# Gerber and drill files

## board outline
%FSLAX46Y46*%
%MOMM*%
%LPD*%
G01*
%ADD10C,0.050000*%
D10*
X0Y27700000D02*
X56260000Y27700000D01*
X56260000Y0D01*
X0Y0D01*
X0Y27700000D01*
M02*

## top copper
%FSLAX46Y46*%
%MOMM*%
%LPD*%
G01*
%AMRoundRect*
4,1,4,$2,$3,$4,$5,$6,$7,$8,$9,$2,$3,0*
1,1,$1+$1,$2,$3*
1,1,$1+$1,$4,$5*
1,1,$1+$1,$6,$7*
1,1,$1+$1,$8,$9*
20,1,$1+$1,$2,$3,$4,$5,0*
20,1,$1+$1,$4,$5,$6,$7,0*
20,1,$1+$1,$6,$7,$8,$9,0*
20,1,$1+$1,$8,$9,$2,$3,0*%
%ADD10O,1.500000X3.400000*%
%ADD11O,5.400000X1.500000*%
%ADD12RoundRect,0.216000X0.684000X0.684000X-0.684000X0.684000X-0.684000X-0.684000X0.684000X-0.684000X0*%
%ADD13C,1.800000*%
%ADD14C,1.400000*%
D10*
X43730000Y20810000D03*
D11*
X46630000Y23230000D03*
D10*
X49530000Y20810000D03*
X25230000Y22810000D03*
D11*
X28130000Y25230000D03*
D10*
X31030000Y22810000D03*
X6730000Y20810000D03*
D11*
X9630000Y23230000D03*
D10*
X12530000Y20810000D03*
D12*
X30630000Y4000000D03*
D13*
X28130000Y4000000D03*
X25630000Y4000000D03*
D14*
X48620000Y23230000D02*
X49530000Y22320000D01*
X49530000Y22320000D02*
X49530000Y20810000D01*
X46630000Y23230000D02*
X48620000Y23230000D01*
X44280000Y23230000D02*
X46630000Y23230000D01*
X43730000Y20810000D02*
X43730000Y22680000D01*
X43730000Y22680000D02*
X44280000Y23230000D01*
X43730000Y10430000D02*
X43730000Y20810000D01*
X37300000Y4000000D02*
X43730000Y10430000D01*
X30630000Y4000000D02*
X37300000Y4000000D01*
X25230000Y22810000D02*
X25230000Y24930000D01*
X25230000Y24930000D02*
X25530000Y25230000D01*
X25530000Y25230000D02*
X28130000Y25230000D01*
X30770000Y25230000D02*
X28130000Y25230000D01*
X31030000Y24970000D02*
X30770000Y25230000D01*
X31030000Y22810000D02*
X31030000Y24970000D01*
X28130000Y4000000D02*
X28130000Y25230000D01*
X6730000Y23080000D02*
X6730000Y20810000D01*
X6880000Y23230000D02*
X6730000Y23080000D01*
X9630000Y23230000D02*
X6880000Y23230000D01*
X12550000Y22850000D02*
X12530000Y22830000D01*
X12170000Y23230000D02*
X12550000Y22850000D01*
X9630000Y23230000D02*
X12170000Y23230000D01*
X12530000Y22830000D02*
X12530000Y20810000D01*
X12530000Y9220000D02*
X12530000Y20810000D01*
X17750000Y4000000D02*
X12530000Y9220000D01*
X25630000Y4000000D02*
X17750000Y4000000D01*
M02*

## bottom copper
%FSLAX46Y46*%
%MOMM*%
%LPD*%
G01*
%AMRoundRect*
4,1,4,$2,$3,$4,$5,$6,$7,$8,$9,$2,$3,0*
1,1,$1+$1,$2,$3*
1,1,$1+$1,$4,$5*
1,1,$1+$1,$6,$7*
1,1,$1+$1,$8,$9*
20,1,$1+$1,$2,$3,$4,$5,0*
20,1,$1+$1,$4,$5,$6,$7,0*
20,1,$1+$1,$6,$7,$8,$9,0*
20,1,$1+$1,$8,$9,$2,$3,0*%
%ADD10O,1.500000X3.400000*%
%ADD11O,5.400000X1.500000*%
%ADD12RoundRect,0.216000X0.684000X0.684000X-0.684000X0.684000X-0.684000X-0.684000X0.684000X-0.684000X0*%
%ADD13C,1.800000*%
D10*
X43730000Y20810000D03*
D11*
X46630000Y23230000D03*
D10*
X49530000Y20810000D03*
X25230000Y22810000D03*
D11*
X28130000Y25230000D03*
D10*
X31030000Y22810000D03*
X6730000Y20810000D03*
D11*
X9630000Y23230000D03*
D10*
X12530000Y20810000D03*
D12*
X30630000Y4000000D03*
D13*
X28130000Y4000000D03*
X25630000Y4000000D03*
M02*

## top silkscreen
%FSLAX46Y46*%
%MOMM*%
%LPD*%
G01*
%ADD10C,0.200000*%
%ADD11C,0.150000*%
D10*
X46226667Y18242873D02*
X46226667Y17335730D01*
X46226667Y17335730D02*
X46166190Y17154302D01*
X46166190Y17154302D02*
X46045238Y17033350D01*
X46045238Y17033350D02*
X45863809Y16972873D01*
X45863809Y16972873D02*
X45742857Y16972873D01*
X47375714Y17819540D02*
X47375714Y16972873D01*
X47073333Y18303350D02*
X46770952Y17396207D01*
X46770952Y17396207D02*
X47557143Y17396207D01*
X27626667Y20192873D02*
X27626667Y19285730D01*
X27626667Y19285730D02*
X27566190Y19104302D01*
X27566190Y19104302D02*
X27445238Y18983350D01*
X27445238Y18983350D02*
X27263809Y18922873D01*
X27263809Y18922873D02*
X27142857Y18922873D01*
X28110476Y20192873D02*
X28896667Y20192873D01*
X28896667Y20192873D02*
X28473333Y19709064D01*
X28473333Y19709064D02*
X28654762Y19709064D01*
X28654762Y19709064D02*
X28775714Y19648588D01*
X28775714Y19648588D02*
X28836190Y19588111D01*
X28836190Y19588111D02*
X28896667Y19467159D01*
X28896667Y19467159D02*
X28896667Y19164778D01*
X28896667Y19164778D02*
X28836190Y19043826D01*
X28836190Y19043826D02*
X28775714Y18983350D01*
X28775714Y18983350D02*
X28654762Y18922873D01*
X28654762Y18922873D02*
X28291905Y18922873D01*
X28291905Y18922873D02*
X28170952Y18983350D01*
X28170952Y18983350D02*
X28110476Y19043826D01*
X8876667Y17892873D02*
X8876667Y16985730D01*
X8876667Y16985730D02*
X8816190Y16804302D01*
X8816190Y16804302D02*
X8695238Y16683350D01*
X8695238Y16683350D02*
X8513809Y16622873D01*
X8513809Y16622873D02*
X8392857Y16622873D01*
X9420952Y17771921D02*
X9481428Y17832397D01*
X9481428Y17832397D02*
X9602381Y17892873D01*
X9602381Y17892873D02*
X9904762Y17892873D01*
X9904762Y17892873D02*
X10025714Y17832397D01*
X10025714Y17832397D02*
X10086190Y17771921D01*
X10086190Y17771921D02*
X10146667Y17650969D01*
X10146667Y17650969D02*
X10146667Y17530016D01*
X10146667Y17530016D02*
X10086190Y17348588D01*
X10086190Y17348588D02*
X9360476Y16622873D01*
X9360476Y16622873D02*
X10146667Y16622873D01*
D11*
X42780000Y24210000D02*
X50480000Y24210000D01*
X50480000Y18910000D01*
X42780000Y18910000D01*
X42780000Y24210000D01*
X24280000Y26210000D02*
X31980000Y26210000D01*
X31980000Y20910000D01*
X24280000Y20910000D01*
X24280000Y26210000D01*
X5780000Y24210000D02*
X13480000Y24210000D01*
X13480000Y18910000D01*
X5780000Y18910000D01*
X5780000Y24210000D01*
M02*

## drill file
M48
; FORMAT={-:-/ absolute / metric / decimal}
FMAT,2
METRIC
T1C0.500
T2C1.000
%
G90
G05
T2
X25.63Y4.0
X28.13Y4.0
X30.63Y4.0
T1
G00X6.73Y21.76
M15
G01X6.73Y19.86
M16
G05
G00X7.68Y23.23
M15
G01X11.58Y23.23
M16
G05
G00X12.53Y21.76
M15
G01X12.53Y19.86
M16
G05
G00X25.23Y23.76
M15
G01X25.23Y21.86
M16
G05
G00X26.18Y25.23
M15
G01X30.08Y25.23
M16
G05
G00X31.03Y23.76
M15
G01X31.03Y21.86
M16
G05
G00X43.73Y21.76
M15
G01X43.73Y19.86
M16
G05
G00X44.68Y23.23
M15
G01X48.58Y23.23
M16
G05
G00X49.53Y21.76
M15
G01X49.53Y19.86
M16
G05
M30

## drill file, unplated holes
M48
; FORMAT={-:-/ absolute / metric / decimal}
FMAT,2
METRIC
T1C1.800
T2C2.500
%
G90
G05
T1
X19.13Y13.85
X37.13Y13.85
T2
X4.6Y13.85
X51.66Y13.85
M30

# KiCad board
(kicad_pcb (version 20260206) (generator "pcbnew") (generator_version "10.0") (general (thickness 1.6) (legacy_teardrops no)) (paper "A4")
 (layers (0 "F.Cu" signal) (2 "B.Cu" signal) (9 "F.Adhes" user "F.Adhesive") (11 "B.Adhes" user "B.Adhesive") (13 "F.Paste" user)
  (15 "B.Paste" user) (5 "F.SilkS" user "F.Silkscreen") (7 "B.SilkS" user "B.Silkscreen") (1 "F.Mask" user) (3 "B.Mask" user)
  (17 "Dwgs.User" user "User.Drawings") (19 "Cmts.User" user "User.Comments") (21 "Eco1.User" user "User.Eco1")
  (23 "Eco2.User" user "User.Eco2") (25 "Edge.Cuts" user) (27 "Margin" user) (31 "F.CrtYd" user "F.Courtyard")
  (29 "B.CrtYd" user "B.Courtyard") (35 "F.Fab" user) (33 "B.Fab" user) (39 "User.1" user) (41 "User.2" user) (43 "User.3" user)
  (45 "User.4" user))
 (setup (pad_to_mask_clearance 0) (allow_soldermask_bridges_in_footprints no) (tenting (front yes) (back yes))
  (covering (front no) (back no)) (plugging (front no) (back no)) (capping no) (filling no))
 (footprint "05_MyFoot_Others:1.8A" (layer "F.Cu") (at 37.13 -13.85)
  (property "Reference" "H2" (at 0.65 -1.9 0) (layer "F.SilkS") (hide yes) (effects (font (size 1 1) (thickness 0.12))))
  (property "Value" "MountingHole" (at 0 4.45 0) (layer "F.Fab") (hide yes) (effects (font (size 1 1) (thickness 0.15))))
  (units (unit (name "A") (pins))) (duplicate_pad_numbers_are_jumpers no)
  (pad "" np_thru_hole circle (at 0 0) (size 1.8 1.8) (drill 1.8) (layers "*.Cu" "*.Mask") (zone_connect 2)))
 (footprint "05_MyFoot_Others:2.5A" (layer "F.Cu") (at 51.66 -13.85)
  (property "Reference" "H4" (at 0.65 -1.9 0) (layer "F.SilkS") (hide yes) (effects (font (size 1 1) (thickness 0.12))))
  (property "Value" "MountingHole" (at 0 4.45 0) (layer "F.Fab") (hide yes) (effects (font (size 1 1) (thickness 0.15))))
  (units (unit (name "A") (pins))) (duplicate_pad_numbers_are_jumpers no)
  (pad "" np_thru_hole circle (at 0 0) (size 2.5 2.5) (drill 2.5) (layers "*.Cu" "*.Mask") (zone_connect 2)))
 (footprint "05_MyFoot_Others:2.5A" (layer "F.Cu") (at 4.6 -13.85)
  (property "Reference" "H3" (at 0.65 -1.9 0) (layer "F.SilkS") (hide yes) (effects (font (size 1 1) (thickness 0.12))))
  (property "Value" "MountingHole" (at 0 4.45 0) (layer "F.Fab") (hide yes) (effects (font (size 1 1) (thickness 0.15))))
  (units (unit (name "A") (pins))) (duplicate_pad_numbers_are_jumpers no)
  (pad "" np_thru_hole circle (at 0 0) (size 2.5 2.5) (drill 2.5) (layers "*.Cu" "*.Mask") (zone_connect 2)))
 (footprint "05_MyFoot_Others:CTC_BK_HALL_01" (layer "F.Cu") (at 28.13 -22.81)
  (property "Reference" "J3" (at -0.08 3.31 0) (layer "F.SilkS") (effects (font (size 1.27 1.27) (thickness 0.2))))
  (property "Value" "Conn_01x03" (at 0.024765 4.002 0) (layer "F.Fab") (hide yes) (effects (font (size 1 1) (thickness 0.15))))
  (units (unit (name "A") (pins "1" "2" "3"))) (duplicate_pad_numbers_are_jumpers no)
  (fp_rect (start -3.85 -3.4) (end 3.85 1.9) (stroke (width 0.15) (type solid)) (fill no) (layer "F.SilkS"))
  (pad "1" thru_hole oval (at -2.9 0) (size 1.5 3.4) (drill oval 0.5 2.4) (layers "*.Cu" "*.Mask") (remove_unused_layers no)
   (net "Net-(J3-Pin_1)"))
  (pad "2" thru_hole oval (at 0 -2.42) (size 5.4 1.5) (drill oval 4.4 0.5) (layers "*.Cu" "*.Mask") (remove_unused_layers no)
   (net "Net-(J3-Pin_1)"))
  (pad "3" thru_hole oval (at 2.9 0) (size 1.5 3.4) (drill oval 0.5 2.4) (layers "*.Cu" "*.Mask") (remove_unused_layers no)
   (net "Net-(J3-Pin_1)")))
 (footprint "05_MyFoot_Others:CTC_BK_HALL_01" (layer "F.Cu") (at 46.63 -20.81)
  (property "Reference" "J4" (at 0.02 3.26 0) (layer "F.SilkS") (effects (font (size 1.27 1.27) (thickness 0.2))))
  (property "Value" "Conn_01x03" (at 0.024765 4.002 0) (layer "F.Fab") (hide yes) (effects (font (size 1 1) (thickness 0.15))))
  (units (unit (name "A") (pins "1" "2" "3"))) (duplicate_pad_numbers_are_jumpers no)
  (fp_rect (start -3.85 -3.4) (end 3.85 1.9) (stroke (width 0.15) (type solid)) (fill no) (layer "F.SilkS"))
  (pad "1" thru_hole oval (at -2.9 0) (size 1.5 3.4) (drill oval 0.5 2.4) (layers "*.Cu" "*.Mask") (remove_unused_layers no)
   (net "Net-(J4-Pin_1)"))
  (pad "2" thru_hole oval (at 0 -2.42) (size 5.4 1.5) (drill oval 4.4 0.5) (layers "*.Cu" "*.Mask") (remove_unused_layers no)
   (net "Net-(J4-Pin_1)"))
  (pad "3" thru_hole oval (at 2.9 0) (size 1.5 3.4) (drill oval 0.5 2.4) (layers "*.Cu" "*.Mask") (remove_unused_layers no)
   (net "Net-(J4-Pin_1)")))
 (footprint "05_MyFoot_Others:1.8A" (layer "F.Cu") (at 19.13 -13.85)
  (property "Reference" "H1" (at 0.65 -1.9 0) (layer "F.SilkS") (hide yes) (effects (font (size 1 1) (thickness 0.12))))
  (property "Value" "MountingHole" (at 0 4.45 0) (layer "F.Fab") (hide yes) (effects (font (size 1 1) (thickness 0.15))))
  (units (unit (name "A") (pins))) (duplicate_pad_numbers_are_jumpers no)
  (pad "" np_thru_hole circle (at 0 0) (size 1.8 1.8) (drill 1.8) (layers "*.Cu" "*.Mask") (zone_connect 2)))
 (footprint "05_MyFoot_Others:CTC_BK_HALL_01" (layer "F.Cu") (at 9.63 -20.81)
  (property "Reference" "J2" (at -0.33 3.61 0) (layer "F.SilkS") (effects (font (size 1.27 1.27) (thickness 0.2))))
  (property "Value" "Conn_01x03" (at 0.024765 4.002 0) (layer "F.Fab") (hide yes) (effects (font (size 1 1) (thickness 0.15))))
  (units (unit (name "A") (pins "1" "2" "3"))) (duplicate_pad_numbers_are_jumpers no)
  (fp_rect (start -3.85 -3.4) (end 3.85 1.9) (stroke (width 0.15) (type solid)) (fill no) (layer "F.SilkS"))
  (pad "1" thru_hole oval (at -2.9 0) (size 1.5 3.4) (drill oval 0.5 2.4) (layers "*.Cu" "*.Mask") (remove_unused_layers no)
   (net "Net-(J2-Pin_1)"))
  (pad "2" thru_hole oval (at 0 -2.42) (size 5.4 1.5) (drill oval 4.4 0.5) (layers "*.Cu" "*.Mask") (remove_unused_layers no)
   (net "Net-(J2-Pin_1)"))
  (pad "3" thru_hole oval (at 2.9 0) (size 1.5 3.4) (drill oval 0.5 2.4) (layers "*.Cu" "*.Mask") (remove_unused_layers no)
   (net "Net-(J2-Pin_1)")))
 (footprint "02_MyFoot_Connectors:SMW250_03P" (layer "B.Cu") (at 28.13 -4 180)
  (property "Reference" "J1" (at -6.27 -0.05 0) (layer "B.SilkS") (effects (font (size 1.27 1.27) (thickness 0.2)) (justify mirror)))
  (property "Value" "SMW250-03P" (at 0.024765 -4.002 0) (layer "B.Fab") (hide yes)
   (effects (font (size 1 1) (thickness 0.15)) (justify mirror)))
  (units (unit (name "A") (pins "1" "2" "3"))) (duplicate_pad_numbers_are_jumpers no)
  (pad "1" thru_hole roundrect (at -2.5 0 180) (size 1.8 1.8) (drill 1) (layers "*.Cu" "*.Mask") (remove_unused_layers no)
   (roundrect_rratio 0.12) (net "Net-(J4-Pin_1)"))
  (pad "2" thru_hole circle (at 0 0 180) (size 1.8 1.8) (drill 1) (layers "*.Cu" "*.Mask") (remove_unused_layers no) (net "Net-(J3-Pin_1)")
   (thermal_bridge_angle 90))
  (pad "3" thru_hole circle (at 2.5 0 180) (size 1.8 1.8) (drill 1) (layers "*.Cu" "*.Mask") (remove_unused_layers no)
   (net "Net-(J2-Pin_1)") (thermal_bridge_angle 90)))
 (gr_rect (start 0 -27.7) (end 56.26 0) (stroke (width 0.05) (type solid)) (fill no) (layer "Edge.Cuts"))
 (segment (start 6.88 -23.23) (end 6.73 -23.08) (width 1.4) (layer "F.Cu") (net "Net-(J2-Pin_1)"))
 (segment (start 12.55 -22.85) (end 12.53 -22.83) (width 1.4) (layer "F.Cu") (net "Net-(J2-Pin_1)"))
 (segment (start 12.53 -22.83) (end 12.53 -20.81) (width 1.4) (layer "F.Cu") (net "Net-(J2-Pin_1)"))
 (segment (start 6.73 -23.08) (end 6.73 -20.81) (width 1.4) (layer "F.Cu") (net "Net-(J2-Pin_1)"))
 (segment (start 9.63 -23.23) (end 6.88 -23.23) (width 1.4) (layer "F.Cu") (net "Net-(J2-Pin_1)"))
 (segment (start 9.63 -23.23) (end 12.17 -23.23) (width 1.4) (layer "F.Cu") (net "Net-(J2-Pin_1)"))
 (segment (start 12.53 -9.22) (end 12.53 -20.81) (width 1.4) (layer "F.Cu") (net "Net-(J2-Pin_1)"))
 (segment (start 17.75 -4) (end 12.53 -9.22) (width 1.4) (layer "F.Cu") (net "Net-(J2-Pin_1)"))
 (segment (start 12.17 -23.23) (end 12.55 -22.85) (width 1.4) (layer "F.Cu") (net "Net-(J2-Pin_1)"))
 (segment (start 25.63 -4) (end 17.75 -4) (width 1.4) (layer "F.Cu") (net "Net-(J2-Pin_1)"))
 (segment (start 31.03 -22.81) (end 31.03 -24.97) (width 1.4) (layer "F.Cu") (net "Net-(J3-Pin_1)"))
 (segment (start 31.03 -24.97) (end 30.77 -25.23) (width 1.4) (layer "F.Cu") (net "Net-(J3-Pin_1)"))
 (segment (start 25.23 -22.81) (end 25.23 -24.93) (width 1.4) (layer "F.Cu") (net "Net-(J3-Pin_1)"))
 (segment (start 25.53 -25.23) (end 28.13 -25.23) (width 1.4) (layer "F.Cu") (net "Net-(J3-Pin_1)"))
 (segment (start 28.13 -4) (end 28.13 -25.23) (width 1.4) (layer "F.Cu") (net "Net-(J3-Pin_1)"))
 (segment (start 30.77 -25.23) (end 28.13 -25.23) (width 1.4) (layer "F.Cu") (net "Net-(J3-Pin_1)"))
 (segment (start 25.23 -24.93) (end 25.53 -25.23) (width 1.4) (layer "F.Cu") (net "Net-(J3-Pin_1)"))
 (segment (start 48.62 -23.23) (end 49.53 -22.32) (width 1.4) (layer "F.Cu") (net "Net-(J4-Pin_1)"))
 (segment (start 43.73 -22.68) (end 44.28 -23.23) (width 1.4) (layer "F.Cu") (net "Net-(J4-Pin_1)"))
 (segment (start 37.3 -4) (end 43.73 -10.43) (width 1.4) (layer "F.Cu") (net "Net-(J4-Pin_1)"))
 (segment (start 49.53 -22.32) (end 49.53 -20.81) (width 1.4) (layer "F.Cu") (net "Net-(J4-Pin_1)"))
 (segment (start 46.63 -23.23) (end 48.62 -23.23) (width 1.4) (layer "F.Cu") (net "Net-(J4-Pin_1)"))
 (segment (start 43.73 -10.43) (end 43.73 -20.81) (width 1.4) (layer "F.Cu") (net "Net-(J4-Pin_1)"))
 (segment (start 43.73 -20.81) (end 43.73 -22.68) (width 1.4) (layer "F.Cu") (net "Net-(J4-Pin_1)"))
 (segment (start 44.28 -23.23) (end 46.63 -23.23) (width 1.4) (layer "F.Cu") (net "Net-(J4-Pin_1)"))
 (segment (start 30.63 -4) (end 37.3 -4) (width 1.4) (layer "F.Cu") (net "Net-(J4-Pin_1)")))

